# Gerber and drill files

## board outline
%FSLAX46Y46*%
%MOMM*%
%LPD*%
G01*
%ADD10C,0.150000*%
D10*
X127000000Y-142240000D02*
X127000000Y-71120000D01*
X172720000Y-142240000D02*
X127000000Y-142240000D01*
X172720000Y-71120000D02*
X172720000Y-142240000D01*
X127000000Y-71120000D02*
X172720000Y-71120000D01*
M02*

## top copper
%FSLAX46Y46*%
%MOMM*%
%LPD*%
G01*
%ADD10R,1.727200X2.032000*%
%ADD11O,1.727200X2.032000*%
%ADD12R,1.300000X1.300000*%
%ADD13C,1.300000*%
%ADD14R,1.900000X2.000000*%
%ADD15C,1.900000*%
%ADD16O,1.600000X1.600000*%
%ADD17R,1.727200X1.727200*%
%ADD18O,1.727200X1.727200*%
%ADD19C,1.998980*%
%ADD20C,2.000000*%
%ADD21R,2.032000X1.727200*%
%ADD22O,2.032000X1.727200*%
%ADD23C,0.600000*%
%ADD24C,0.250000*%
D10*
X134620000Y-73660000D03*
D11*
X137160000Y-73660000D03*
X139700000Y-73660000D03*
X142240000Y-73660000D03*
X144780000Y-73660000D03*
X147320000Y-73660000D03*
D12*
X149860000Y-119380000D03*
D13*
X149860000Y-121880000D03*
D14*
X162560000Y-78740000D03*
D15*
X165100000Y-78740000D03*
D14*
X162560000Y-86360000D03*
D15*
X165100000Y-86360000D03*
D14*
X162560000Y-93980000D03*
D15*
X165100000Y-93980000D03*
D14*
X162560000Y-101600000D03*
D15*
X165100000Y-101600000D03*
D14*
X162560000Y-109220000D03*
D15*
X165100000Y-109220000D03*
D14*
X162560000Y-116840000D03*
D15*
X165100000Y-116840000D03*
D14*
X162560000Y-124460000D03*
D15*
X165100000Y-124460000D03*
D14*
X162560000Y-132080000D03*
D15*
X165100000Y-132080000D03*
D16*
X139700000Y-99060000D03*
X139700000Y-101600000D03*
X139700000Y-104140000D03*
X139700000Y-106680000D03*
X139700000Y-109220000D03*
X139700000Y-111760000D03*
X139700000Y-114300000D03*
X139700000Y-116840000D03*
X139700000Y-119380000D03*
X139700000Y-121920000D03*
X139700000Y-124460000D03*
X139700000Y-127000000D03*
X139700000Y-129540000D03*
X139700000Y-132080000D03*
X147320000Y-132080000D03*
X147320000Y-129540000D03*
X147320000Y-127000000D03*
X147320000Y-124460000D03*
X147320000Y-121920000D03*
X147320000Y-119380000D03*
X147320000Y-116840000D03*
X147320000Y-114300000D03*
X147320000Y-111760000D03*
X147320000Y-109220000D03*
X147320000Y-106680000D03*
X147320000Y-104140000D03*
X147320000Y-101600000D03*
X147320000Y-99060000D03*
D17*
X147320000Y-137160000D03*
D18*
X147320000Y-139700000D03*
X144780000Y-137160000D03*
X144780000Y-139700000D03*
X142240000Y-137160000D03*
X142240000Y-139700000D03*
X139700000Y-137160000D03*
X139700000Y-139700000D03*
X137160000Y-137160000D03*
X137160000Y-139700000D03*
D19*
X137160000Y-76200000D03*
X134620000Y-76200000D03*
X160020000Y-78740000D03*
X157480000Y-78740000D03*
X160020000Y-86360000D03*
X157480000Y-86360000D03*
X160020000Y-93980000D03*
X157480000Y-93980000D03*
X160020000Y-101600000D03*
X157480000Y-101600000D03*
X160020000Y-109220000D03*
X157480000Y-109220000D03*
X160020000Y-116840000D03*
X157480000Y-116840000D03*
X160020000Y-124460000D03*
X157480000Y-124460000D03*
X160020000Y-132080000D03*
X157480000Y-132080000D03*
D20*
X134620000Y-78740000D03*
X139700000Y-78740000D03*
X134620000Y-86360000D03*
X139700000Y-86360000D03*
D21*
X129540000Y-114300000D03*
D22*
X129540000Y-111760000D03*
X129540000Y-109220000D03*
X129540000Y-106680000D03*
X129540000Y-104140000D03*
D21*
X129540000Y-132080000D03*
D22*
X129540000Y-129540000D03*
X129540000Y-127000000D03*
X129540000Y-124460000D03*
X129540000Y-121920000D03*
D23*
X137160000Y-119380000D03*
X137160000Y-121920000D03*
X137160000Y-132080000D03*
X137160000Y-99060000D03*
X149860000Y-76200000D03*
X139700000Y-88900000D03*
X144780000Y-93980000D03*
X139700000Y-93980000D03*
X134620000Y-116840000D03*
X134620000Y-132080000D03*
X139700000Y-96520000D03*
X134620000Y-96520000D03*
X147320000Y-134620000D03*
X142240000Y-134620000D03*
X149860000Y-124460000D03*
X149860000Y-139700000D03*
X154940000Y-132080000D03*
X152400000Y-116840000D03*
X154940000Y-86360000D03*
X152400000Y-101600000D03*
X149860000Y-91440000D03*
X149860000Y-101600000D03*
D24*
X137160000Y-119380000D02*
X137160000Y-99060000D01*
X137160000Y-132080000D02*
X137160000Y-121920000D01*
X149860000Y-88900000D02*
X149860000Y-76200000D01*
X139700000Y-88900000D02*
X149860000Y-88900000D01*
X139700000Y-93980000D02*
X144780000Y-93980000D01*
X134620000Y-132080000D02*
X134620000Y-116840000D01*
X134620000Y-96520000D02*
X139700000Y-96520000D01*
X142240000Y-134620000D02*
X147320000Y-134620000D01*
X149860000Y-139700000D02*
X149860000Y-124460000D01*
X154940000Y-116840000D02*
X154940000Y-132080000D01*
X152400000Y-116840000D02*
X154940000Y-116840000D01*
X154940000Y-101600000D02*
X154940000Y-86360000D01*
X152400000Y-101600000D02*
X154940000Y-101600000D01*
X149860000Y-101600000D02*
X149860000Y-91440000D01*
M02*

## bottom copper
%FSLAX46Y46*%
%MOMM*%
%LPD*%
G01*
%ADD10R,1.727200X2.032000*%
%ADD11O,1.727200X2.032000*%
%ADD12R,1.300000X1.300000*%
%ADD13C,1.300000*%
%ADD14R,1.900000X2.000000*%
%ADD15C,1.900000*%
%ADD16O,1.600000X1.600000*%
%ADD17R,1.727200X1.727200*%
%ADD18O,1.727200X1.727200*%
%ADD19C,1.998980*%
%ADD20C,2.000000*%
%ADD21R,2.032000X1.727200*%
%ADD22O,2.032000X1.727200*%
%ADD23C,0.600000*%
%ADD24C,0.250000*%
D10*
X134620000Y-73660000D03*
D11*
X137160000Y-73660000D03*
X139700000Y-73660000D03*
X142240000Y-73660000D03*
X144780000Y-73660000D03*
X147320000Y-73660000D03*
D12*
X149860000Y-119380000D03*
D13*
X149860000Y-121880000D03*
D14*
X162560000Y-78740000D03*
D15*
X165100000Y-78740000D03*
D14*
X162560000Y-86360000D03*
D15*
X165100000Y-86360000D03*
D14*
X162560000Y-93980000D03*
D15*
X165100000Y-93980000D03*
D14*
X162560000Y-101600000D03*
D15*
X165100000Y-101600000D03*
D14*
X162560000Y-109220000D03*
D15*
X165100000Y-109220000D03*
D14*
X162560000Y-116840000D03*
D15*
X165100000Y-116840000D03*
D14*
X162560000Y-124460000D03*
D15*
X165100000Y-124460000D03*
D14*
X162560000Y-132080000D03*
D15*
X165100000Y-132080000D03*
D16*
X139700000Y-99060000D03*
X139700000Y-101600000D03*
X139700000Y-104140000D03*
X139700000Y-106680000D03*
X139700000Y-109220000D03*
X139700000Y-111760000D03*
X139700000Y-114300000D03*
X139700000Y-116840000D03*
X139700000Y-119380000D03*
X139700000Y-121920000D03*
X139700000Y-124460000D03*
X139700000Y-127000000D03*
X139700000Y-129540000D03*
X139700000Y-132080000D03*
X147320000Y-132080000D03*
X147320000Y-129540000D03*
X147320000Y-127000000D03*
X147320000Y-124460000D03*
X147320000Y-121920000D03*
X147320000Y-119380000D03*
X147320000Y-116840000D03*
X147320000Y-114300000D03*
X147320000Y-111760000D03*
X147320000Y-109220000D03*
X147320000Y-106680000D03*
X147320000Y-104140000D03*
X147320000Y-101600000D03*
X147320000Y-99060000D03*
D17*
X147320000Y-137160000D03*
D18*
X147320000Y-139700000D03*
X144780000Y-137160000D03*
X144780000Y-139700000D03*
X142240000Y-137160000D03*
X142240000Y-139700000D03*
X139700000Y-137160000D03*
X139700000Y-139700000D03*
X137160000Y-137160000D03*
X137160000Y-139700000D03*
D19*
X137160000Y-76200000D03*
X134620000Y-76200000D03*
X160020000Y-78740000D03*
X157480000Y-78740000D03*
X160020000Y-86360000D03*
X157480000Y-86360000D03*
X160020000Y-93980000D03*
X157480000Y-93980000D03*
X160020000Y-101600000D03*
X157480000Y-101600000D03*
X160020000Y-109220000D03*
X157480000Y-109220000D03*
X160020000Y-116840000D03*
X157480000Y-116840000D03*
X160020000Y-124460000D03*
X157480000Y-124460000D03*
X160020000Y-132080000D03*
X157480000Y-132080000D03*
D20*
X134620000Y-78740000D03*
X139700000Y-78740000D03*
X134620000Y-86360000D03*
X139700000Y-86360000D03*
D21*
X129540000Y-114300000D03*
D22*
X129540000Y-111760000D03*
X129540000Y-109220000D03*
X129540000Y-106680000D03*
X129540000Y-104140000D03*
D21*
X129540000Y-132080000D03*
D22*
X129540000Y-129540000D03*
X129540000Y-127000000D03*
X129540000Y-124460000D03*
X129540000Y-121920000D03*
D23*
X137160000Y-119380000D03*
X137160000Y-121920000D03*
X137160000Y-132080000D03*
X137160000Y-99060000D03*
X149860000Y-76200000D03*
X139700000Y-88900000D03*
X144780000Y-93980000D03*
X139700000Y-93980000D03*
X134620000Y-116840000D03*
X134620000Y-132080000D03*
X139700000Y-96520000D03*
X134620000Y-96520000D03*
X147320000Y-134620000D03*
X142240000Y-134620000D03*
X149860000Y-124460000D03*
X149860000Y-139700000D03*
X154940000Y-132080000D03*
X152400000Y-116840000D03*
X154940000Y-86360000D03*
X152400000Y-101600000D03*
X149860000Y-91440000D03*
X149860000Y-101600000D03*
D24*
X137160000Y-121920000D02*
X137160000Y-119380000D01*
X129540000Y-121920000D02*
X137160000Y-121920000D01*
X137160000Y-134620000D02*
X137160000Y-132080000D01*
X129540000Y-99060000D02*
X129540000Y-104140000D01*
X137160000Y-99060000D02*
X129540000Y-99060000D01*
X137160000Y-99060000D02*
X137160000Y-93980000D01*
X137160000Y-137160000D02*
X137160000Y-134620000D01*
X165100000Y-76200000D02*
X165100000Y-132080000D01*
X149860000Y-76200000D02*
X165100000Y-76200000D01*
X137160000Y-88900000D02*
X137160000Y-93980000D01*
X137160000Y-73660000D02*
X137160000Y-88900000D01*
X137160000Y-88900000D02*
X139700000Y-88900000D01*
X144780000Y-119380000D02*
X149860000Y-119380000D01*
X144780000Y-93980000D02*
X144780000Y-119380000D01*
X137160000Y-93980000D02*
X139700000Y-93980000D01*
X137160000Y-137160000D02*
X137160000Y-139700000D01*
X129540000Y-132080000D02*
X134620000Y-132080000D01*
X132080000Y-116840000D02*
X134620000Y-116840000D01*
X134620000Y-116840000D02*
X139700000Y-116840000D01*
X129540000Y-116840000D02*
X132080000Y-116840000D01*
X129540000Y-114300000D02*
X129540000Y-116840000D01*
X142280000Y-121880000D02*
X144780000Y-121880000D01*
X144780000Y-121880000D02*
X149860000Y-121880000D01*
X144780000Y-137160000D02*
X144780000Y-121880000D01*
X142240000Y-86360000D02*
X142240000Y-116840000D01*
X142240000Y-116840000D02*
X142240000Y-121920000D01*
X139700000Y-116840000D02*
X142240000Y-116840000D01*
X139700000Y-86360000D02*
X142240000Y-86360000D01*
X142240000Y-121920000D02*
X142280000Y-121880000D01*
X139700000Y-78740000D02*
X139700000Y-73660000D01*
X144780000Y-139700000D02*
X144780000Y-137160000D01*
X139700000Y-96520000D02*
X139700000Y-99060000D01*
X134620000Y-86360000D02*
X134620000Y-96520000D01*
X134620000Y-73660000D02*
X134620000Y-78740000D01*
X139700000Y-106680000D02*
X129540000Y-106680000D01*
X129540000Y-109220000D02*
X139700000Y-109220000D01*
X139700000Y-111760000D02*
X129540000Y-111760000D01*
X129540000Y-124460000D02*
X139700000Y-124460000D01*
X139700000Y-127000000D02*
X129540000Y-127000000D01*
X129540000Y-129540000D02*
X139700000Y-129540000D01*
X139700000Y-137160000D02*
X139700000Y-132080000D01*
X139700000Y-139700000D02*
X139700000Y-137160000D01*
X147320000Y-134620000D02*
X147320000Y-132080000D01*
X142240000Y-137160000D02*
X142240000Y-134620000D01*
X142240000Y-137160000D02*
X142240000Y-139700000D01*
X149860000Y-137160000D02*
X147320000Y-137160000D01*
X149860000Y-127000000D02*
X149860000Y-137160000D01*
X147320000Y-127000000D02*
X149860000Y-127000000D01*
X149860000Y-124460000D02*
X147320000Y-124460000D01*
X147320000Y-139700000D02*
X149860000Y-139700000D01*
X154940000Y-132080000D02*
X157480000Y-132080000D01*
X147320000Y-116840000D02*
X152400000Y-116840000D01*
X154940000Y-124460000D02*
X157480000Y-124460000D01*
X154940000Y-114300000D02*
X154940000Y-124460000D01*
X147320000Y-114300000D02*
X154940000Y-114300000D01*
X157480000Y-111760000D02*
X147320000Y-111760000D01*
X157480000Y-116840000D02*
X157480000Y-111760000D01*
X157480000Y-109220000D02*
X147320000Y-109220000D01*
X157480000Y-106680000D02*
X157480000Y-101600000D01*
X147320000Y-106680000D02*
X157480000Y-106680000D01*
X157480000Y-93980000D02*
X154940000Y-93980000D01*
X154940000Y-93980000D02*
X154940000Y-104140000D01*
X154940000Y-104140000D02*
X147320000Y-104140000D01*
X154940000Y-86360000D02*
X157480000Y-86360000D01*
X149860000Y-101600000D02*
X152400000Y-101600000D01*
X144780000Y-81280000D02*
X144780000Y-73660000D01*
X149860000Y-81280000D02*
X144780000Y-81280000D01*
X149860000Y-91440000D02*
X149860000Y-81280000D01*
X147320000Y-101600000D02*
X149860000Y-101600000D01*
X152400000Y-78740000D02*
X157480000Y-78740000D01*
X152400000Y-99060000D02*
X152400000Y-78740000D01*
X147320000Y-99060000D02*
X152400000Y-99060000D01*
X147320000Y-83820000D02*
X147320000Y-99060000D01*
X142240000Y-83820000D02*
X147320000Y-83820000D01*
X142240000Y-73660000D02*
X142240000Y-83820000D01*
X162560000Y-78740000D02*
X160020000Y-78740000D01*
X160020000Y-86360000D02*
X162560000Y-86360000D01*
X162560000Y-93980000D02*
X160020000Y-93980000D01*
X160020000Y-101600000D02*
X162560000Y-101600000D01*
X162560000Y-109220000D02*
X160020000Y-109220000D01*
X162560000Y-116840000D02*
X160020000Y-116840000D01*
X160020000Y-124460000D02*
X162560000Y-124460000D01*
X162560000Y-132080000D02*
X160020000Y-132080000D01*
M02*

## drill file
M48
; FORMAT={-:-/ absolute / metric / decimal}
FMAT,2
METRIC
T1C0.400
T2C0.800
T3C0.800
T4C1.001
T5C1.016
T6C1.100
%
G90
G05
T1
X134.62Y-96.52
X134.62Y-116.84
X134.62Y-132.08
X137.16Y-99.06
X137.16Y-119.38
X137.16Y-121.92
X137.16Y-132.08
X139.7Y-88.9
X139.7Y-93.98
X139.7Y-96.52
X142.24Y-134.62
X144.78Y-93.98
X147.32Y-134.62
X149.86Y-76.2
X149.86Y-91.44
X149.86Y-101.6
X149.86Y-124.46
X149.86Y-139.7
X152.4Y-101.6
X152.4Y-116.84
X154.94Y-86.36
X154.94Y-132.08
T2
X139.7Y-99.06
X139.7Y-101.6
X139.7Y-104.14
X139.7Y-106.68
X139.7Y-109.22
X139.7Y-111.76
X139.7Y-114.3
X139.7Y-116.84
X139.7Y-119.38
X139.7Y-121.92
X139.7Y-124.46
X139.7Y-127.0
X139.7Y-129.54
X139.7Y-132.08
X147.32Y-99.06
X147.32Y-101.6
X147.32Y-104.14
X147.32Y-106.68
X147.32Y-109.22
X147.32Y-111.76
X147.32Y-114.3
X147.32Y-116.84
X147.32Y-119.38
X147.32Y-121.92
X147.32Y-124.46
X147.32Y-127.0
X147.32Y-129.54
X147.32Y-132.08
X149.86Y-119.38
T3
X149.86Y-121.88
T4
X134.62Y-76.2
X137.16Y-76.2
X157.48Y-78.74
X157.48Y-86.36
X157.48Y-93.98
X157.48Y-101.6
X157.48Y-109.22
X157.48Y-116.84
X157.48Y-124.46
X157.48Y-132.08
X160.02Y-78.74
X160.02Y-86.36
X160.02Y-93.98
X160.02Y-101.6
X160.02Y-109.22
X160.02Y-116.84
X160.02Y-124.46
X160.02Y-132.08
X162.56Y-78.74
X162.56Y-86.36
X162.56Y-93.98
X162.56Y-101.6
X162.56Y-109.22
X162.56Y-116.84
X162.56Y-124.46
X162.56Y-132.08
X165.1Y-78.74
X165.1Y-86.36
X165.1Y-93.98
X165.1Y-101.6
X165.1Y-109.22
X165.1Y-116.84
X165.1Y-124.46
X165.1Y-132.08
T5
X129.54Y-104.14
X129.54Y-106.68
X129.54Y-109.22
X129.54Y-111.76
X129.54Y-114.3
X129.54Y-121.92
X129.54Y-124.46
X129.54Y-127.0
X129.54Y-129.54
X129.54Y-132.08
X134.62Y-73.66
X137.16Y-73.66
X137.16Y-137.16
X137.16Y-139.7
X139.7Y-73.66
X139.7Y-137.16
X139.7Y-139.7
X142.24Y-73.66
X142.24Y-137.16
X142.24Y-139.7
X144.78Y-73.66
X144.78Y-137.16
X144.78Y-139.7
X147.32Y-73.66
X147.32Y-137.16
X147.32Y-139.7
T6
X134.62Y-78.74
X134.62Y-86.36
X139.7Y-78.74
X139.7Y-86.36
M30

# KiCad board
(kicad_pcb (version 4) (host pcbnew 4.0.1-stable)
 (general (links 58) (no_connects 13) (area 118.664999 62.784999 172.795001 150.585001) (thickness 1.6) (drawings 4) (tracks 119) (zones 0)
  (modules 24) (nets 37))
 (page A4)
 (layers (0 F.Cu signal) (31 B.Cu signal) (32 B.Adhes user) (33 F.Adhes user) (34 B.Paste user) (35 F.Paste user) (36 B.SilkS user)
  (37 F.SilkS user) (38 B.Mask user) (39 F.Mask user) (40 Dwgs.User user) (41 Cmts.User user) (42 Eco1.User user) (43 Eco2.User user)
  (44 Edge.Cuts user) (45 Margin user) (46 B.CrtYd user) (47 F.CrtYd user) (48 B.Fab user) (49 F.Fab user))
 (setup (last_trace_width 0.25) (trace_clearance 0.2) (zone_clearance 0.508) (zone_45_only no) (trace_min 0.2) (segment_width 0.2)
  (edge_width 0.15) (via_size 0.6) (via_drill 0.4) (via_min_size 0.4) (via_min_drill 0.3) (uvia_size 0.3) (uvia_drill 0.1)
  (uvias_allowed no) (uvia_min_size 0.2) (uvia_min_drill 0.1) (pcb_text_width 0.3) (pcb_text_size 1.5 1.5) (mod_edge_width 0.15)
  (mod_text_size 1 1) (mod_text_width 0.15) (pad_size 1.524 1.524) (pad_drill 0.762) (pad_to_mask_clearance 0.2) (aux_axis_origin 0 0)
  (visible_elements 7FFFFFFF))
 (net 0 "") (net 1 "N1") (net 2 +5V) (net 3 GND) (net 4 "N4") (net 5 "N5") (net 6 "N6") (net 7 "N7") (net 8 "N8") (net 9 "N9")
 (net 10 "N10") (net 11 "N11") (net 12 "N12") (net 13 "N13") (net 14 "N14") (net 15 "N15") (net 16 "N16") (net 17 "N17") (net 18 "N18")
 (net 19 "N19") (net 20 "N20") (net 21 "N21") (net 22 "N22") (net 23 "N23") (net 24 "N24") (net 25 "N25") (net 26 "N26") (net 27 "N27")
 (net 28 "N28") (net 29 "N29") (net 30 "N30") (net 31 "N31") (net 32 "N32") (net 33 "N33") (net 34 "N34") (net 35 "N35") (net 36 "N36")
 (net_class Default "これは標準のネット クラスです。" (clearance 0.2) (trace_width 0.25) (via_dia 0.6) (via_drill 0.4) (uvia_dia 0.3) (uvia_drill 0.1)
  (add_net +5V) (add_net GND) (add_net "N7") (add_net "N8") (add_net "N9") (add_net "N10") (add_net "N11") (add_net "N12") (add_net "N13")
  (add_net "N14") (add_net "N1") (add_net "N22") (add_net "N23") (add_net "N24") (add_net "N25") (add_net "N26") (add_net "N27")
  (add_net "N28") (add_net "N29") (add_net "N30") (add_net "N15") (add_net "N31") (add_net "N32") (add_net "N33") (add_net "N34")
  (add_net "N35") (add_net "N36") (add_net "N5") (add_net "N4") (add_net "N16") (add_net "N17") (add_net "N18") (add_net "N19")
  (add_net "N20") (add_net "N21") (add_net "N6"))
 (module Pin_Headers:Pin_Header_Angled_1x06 (layer F.Cu) (at 134.62 73.66 90)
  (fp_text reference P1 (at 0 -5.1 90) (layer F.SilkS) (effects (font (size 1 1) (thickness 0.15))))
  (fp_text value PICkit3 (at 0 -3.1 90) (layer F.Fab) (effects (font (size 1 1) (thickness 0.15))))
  (pad 1 thru_hole rect (at 0 0 90) (size 2.032 1.7272) (drill 1.016) (layers *.Cu *.Mask) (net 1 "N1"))
  (pad 2 thru_hole oval (at 0 2.54 90) (size 2.032 1.7272) (drill 1.016) (layers *.Cu *.Mask) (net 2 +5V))
  (pad 3 thru_hole oval (at 0 5.08 90) (size 2.032 1.7272) (drill 1.016) (layers *.Cu *.Mask) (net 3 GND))
  (pad 4 thru_hole oval (at 0 7.62 90) (size 2.032 1.7272) (drill 1.016) (layers *.Cu *.Mask) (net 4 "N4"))
  (pad 5 thru_hole oval (at 0 10.16 90) (size 2.032 1.7272) (drill 1.016) (layers *.Cu *.Mask) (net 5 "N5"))
  (pad 6 thru_hole oval (at 0 12.7 90) (size 2.032 1.7272) (drill 1.016) (layers *.Cu *.Mask) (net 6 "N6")))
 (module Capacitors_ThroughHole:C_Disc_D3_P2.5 (layer F.Cu) (at 149.86 119.38 270)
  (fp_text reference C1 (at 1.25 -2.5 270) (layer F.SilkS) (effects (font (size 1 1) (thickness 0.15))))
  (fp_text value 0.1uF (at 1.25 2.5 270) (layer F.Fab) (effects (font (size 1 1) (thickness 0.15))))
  (pad 1 thru_hole rect (at 0 0 270) (size 1.3 1.3) (drill 0.8) (layers *.Cu *.Mask) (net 2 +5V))
  (pad 2 thru_hole circle (at 2.5 0 270) (size 1.3 1.3) (drill 0.8001) (layers *.Cu *.Mask) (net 3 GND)))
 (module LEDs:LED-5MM (layer F.Cu) (at 162.56 78.74)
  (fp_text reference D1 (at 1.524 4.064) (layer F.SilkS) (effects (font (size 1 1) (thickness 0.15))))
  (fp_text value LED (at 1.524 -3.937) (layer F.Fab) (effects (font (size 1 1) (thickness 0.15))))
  (pad 1 thru_hole rect (at 0 0 90) (size 2 1.9) (drill 1.00076) (layers *.Cu *.Mask) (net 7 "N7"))
  (pad 2 thru_hole circle (at 2.54 0) (size 1.9 1.9) (drill 1.00076) (layers *.Cu *.Mask) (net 2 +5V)))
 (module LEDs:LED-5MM (layer F.Cu) (at 162.56 86.36)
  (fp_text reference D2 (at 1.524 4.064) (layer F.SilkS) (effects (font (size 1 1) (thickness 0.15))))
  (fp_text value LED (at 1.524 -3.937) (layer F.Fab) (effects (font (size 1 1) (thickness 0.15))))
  (pad 1 thru_hole rect (at 0 0 90) (size 2 1.9) (drill 1.00076) (layers *.Cu *.Mask) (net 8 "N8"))
  (pad 2 thru_hole circle (at 2.54 0) (size 1.9 1.9) (drill 1.00076) (layers *.Cu *.Mask) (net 2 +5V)))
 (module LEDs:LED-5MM (layer F.Cu) (at 162.56 93.98)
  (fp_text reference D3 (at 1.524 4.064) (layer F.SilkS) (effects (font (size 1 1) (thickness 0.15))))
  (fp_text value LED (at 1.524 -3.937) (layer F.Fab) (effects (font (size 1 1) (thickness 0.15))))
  (pad 1 thru_hole rect (at 0 0 90) (size 2 1.9) (drill 1.00076) (layers *.Cu *.Mask) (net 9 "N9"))
  (pad 2 thru_hole circle (at 2.54 0) (size 1.9 1.9) (drill 1.00076) (layers *.Cu *.Mask) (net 2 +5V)))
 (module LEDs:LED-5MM (layer F.Cu) (at 162.56 101.6)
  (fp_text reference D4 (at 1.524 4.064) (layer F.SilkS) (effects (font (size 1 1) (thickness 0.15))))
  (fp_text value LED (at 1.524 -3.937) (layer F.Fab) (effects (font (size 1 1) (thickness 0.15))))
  (pad 1 thru_hole rect (at 0 0 90) (size 2 1.9) (drill 1.00076) (layers *.Cu *.Mask) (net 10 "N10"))
  (pad 2 thru_hole circle (at 2.54 0) (size 1.9 1.9) (drill 1.00076) (layers *.Cu *.Mask) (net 2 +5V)))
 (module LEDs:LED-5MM (layer F.Cu) (at 162.56 109.22)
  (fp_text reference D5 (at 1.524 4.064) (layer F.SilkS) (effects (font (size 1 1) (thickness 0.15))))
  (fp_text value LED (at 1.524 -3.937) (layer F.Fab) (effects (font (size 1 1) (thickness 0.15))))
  (pad 1 thru_hole rect (at 0 0 90) (size 2 1.9) (drill 1.00076) (layers *.Cu *.Mask) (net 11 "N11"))
  (pad 2 thru_hole circle (at 2.54 0) (size 1.9 1.9) (drill 1.00076) (layers *.Cu *.Mask) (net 2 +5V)))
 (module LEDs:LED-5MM (layer F.Cu) (at 162.56 116.84)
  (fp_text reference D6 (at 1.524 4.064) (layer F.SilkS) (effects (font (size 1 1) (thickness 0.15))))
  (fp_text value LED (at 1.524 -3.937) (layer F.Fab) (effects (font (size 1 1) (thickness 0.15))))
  (pad 1 thru_hole rect (at 0 0 90) (size 2 1.9) (drill 1.00076) (layers *.Cu *.Mask) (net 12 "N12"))
  (pad 2 thru_hole circle (at 2.54 0) (size 1.9 1.9) (drill 1.00076) (layers *.Cu *.Mask) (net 2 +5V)))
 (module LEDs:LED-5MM (layer F.Cu) (at 162.56 124.46)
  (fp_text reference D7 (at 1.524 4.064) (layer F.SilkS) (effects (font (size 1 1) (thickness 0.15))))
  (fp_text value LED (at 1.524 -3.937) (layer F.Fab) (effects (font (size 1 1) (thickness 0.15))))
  (pad 1 thru_hole rect (at 0 0 90) (size 2 1.9) (drill 1.00076) (layers *.Cu *.Mask) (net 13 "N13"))
  (pad 2 thru_hole circle (at 2.54 0) (size 1.9 1.9) (drill 1.00076) (layers *.Cu *.Mask) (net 2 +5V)))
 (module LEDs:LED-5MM (layer F.Cu) (at 162.56 132.08)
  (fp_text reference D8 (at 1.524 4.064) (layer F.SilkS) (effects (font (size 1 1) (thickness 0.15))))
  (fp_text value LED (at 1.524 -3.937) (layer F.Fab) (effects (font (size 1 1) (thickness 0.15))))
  (pad 1 thru_hole rect (at 0 0 90) (size 2 1.9) (drill 1.00076) (layers *.Cu *.Mask) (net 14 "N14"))
  (pad 2 thru_hole circle (at 2.54 0) (size 1.9 1.9) (drill 1.00076) (layers *.Cu *.Mask) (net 2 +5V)))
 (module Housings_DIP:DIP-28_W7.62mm (layer F.Cu) (at 139.7 99.06)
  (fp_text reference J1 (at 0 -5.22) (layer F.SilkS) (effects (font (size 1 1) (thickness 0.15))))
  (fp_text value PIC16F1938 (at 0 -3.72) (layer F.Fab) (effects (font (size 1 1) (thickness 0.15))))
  (pad 1 thru_hole oval (at 0 0) (size 1.6 1.6) (drill 0.8) (layers *.Cu *.Mask) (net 1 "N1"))
  (pad 2 thru_hole oval (at 0 2.54) (size 1.6 1.6) (drill 0.8) (layers *.Cu *.Mask) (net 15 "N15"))
  (pad 3 thru_hole oval (at 0 5.08) (size 1.6 1.6) (drill 0.8) (layers *.Cu *.Mask) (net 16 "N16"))
  (pad 4 thru_hole oval (at 0 7.62) (size 1.6 1.6) (drill 0.8) (layers *.Cu *.Mask) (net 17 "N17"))
  (pad 5 thru_hole oval (at 0 10.16) (size 1.6 1.6) (drill 0.8) (layers *.Cu *.Mask) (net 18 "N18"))
  (pad 6 thru_hole oval (at 0 12.7) (size 1.6 1.6) (drill 0.8) (layers *.Cu *.Mask) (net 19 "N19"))
  (pad 7 thru_hole oval (at 0 15.24) (size 1.6 1.6) (drill 0.8) (layers *.Cu *.Mask) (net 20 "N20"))
  (pad 8 thru_hole oval (at 0 17.78) (size 1.6 1.6) (drill 0.8) (layers *.Cu *.Mask) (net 3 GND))
  (pad 9 thru_hole oval (at 0 20.32) (size 1.6 1.6) (drill 0.8) (layers *.Cu *.Mask) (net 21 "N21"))
  (pad 10 thru_hole oval (at 0 22.86) (size 1.6 1.6) (drill 0.8) (layers *.Cu *.Mask) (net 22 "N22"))
  (pad 11 thru_hole oval (at 0 25.4) (size 1.6 1.6) (drill 0.8) (layers *.Cu *.Mask) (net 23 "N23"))
  (pad 12 thru_hole oval (at 0 27.94) (size 1.6 1.6) (drill 0.8) (layers *.Cu *.Mask) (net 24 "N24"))
  (pad 13 thru_hole oval (at 0 30.48) (size 1.6 1.6) (drill 0.8) (layers *.Cu *.Mask) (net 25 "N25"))
  (pad 14 thru_hole oval (at 0 33.02) (size 1.6 1.6) (drill 0.8) (layers *.Cu *.Mask) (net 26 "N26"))
  (pad 15 thru_hole oval (at 7.62 33.02) (size 1.6 1.6) (drill 0.8) (layers *.Cu *.Mask) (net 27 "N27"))
  (pad 16 thru_hole oval (at 7.62 30.48) (size 1.6 1.6) (drill 0.8) (layers *.Cu *.Mask) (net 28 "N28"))
  (pad 17 thru_hole oval (at 7.62 27.94) (size 1.6 1.6) (drill 0.8) (layers *.Cu *.Mask) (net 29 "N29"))
  (pad 18 thru_hole oval (at 7.62 25.4) (size 1.6 1.6) (drill 0.8) (layers *.Cu *.Mask) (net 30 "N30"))
  (pad 19 thru_hole oval (at 7.62 22.86) (size 1.6 1.6) (drill 0.8) (layers *.Cu *.Mask) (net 3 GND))
  (pad 20 thru_hole oval (at 7.62 20.32) (size 1.6 1.6) (drill 0.8) (layers *.Cu *.Mask) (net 2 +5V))
  (pad 21 thru_hole oval (at 7.62 17.78) (size 1.6 1.6) (drill 0.8) (layers *.Cu *.Mask) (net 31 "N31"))
  (pad 22 thru_hole oval (at 7.62 15.24) (size 1.6 1.6) (drill 0.8) (layers *.Cu *.Mask) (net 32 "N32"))
  (pad 23 thru_hole oval (at 7.62 12.7) (size 1.6 1.6) (drill 0.8) (layers *.Cu *.Mask) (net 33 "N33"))
  (pad 24 thru_hole oval (at 7.62 10.16) (size 1.6 1.6) (drill 0.8) (layers *.Cu *.Mask) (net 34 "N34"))
  (pad 25 thru_hole oval (at 7.62 7.62) (size 1.6 1.6) (drill 0.8) (layers *.Cu *.Mask) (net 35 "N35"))
  (pad 26 thru_hole oval (at 7.62 5.08) (size 1.6 1.6) (drill 0.8) (layers *.Cu *.Mask) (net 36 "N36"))
  (pad 27 thru_hole oval (at 7.62 2.54) (size 1.6 1.6) (drill 0.8) (layers *.Cu *.Mask) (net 5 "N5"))
  (pad 28 thru_hole oval (at 7.62 0) (size 1.6 1.6) (drill 0.8) (layers *.Cu *.Mask) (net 4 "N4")))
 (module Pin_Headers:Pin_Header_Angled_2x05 (layer F.Cu) (at 147.32 137.16 270)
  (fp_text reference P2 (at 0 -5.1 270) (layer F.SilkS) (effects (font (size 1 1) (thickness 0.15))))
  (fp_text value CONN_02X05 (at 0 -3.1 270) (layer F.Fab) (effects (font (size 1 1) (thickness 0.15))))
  (pad 1 thru_hole rect (at 0 0 270) (size 1.7272 1.7272) (drill 1.016) (layers *.Cu *.Mask) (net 29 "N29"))
  (pad 2 thru_hole oval (at 2.54 0 270) (size 1.7272 1.7272) (drill 1.016) (layers *.Cu *.Mask) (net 30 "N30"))
  (pad 3 thru_hole oval (at 0 2.54 270) (size 1.7272 1.7272) (drill 1.016) (layers *.Cu *.Mask) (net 3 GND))
  (pad 4 thru_hole oval (at 2.54 2.54 270) (size 1.7272 1.7272) (drill 1.016) (layers *.Cu *.Mask) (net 3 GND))
  (pad 5 thru_hole oval (at 0 5.08 270) (size 1.7272 1.7272) (drill 1.016) (layers *.Cu *.Mask) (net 27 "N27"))
  (pad 6 thru_hole oval (at 2.54 5.08 270) (size 1.7272 1.7272) (drill 1.016) (layers *.Cu *.Mask) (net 27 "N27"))
  (pad 7 thru_hole oval (at 0 7.62 270) (size 1.7272 1.7272) (drill 1.016) (layers *.Cu *.Mask) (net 26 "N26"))
  (pad 8 thru_hole oval (at 2.54 7.62 270) (size 1.7272 1.7272) (drill 1.016) (layers *.Cu *.Mask) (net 26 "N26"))
  (pad 9 thru_hole oval (at 0 10.16 270) (size 1.7272 1.7272) (drill 1.016) (layers *.Cu *.Mask) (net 2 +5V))
  (pad 10 thru_hole oval (at 2.54 10.16 270) (size 1.7272 1.7272) (drill 1.016) (layers *.Cu *.Mask) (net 2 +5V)))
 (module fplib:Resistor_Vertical (layer F.Cu) (at 135.89 76.2 180)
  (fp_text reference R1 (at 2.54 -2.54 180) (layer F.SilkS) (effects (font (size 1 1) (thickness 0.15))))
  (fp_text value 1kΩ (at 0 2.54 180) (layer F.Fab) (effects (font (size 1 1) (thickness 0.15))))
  (pad 1 thru_hole circle (at -1.27 0 180) (size 1.99898 1.99898) (drill 1.00076) (layers *.Cu *.SilkS *.Mask) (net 2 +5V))
  (pad 2 thru_hole circle (at 1.27 0 180) (size 1.99898 1.99898) (drill 1.00076) (layers *.Cu *.SilkS *.Mask) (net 1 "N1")))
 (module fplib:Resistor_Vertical (layer F.Cu) (at 158.75 78.74 180)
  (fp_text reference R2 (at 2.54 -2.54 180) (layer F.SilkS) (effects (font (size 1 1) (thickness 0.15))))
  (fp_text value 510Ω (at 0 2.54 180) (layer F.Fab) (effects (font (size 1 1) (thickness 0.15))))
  (pad 1 thru_hole circle (at -1.27 0 180) (size 1.99898 1.99898) (drill 1.00076) (layers *.Cu *.SilkS *.Mask) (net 7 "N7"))
  (pad 2 thru_hole circle (at 1.27 0 180) (size 1.99898 1.99898) (drill 1.00076) (layers *.Cu *.SilkS *.Mask) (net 4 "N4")))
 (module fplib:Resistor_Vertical (layer F.Cu) (at 158.75 86.36 180)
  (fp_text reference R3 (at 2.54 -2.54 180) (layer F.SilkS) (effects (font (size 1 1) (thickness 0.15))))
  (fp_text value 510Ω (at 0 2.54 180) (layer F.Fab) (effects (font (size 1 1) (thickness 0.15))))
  (pad 1 thru_hole circle (at -1.27 0 180) (size 1.99898 1.99898) (drill 1.00076) (layers *.Cu *.SilkS *.Mask) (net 8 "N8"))
  (pad 2 thru_hole circle (at 1.27 0 180) (size 1.99898 1.99898) (drill 1.00076) (layers *.Cu *.SilkS *.Mask) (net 5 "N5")))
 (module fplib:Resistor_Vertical (layer F.Cu) (at 158.75 93.98 180)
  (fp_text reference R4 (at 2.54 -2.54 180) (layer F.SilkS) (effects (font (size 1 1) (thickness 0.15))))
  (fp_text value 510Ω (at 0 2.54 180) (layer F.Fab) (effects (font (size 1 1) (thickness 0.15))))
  (pad 1 thru_hole circle (at -1.27 0 180) (size 1.99898 1.99898) (drill 1.00076) (layers *.Cu *.SilkS *.Mask) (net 9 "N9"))
  (pad 2 thru_hole circle (at 1.27 0 180) (size 1.99898 1.99898) (drill 1.00076) (layers *.Cu *.SilkS *.Mask) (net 36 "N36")))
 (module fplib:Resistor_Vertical (layer F.Cu) (at 158.75 101.6 180)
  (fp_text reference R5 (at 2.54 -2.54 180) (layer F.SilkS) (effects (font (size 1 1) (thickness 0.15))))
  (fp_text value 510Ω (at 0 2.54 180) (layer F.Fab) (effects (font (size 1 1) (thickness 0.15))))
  (pad 1 thru_hole circle (at -1.27 0 180) (size 1.99898 1.99898) (drill 1.00076) (layers *.Cu *.SilkS *.Mask) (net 10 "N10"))
  (pad 2 thru_hole circle (at 1.27 0 180) (size 1.99898 1.99898) (drill 1.00076) (layers *.Cu *.SilkS *.Mask) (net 35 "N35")))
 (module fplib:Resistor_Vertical (layer F.Cu) (at 158.75 109.22 180)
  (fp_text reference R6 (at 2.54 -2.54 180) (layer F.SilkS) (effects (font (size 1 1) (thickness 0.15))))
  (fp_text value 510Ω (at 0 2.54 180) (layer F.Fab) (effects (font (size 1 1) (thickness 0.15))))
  (pad 1 thru_hole circle (at -1.27 0 180) (size 1.99898 1.99898) (drill 1.00076) (layers *.Cu *.SilkS *.Mask) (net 11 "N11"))
  (pad 2 thru_hole circle (at 1.27 0 180) (size 1.99898 1.99898) (drill 1.00076) (layers *.Cu *.SilkS *.Mask) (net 34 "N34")))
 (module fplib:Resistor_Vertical (layer F.Cu) (at 158.75 116.84 180)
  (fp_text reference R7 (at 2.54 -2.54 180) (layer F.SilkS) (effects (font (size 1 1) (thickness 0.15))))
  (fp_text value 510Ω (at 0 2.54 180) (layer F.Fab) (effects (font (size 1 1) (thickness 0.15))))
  (pad 1 thru_hole circle (at -1.27 0 180) (size 1.99898 1.99898) (drill 1.00076) (layers *.Cu *.SilkS *.Mask) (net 12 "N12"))
  (pad 2 thru_hole circle (at 1.27 0 180) (size 1.99898 1.99898) (drill 1.00076) (layers *.Cu *.SilkS *.Mask) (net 33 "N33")))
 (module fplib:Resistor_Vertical (layer F.Cu) (at 158.75 124.46 180)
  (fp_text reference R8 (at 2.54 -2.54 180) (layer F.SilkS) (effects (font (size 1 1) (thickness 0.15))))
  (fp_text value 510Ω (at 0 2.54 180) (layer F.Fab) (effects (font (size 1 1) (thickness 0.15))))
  (pad 1 thru_hole circle (at -1.27 0 180) (size 1.99898 1.99898) (drill 1.00076) (layers *.Cu *.SilkS *.Mask) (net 13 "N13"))
  (pad 2 thru_hole circle (at 1.27 0 180) (size 1.99898 1.99898) (drill 1.00076) (layers *.Cu *.SilkS *.Mask) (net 32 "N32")))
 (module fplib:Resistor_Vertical (layer F.Cu) (at 158.75 132.08 180)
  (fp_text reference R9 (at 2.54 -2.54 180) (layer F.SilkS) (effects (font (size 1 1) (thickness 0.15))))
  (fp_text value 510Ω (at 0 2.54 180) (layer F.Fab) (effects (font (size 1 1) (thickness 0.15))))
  (pad 1 thru_hole circle (at -1.27 0 180) (size 1.99898 1.99898) (drill 1.00076) (layers *.Cu *.SilkS *.Mask) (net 14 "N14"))
  (pad 2 thru_hole circle (at 1.27 0 180) (size 1.99898 1.99898) (drill 1.00076) (layers *.Cu *.SilkS *.Mask) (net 31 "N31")))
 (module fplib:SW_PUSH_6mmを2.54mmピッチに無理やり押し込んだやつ (layer F.Cu) (at 137.16 82.55 270)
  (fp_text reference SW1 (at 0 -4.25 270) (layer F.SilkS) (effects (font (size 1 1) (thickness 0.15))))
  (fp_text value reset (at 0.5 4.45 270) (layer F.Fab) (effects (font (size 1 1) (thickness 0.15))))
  (pad 2 thru_hole circle (at -3.81 2.54) (size 2 2) (drill 1.1) (layers *.Cu *.Mask) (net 1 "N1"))
  (pad 1 thru_hole circle (at -3.81 -2.54) (size 2 2) (drill 1.1) (layers *.Cu *.Mask) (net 3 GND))
  (pad 2 thru_hole circle (at 3.81 2.54) (size 2 2) (drill 1.1) (layers *.Cu *.Mask) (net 1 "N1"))
  (pad 1 thru_hole circle (at 3.81 -2.54) (size 2 2) (drill 1.1) (layers *.Cu *.Mask) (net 3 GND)))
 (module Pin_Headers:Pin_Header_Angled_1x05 (layer F.Cu) (at 129.54 114.3 180)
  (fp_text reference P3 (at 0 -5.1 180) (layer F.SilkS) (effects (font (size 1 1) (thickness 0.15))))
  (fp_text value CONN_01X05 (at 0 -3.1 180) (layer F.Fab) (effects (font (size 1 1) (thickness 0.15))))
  (pad 1 thru_hole rect (at 0 0 180) (size 2.032 1.7272) (drill 1.016) (layers *.Cu *.Mask F.SilkS) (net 3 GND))
  (pad 2 thru_hole oval (at 0 2.54 180) (size 2.032 1.7272) (drill 1.016) (layers *.Cu *.Mask F.SilkS) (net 19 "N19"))
  (pad 3 thru_hole oval (at 0 5.08 180) (size 2.032 1.7272) (drill 1.016) (layers *.Cu *.Mask F.SilkS) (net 18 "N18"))
  (pad 4 thru_hole oval (at 0 7.62 180) (size 2.032 1.7272) (drill 1.016) (layers *.Cu *.Mask F.SilkS) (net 17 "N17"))
  (pad 5 thru_hole oval (at 0 10.16 180) (size 2.032 1.7272) (drill 1.016) (layers *.Cu *.Mask F.SilkS) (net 2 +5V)))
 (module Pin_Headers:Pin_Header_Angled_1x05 (layer F.Cu) (at 129.54 132.08 180)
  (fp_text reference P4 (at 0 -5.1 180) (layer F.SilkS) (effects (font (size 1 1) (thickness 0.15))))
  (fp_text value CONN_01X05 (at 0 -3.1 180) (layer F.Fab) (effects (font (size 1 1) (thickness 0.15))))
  (pad 1 thru_hole rect (at 0 0 180) (size 2.032 1.7272) (drill 1.016) (layers *.Cu *.Mask F.SilkS) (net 3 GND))
  (pad 2 thru_hole oval (at 0 2.54 180) (size 2.032 1.7272) (drill 1.016) (layers *.Cu *.Mask F.SilkS) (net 25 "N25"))
  (pad 3 thru_hole oval (at 0 5.08 180) (size 2.032 1.7272) (drill 1.016) (layers *.Cu *.Mask F.SilkS) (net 24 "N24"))
  (pad 4 thru_hole oval (at 0 7.62 180) (size 2.032 1.7272) (drill 1.016) (layers *.Cu *.Mask F.SilkS) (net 23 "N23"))
  (pad 5 thru_hole oval (at 0 10.16 180) (size 2.032 1.7272) (drill 1.016) (layers *.Cu *.Mask F.SilkS) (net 2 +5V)))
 (gr_line (start 127 142.24) (end 127 71.12) (layer Edge.Cuts) (width 0.15))
 (gr_line (start 172.72 142.24) (end 127 142.24) (layer Edge.Cuts) (width 0.15))
 (gr_line (start 172.72 71.12) (end 172.72 142.24) (layer Edge.Cuts) (width 0.15))
 (gr_line (start 127 71.12) (end 172.72 71.12) (layer Edge.Cuts) (width 0.15))
 (segment (start 137.16 121.92) (end 137.16 119.38) (width 0.25) (layer B.Cu) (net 2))
 (via (at 137.16 119.38) (size 0.6) (drill 0.4) (layers F.Cu B.Cu) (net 2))
 (segment (start 129.54 121.92) (end 137.16 121.92) (width 0.25) (layer B.Cu) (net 2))
 (segment (start 137.16 119.38) (end 137.16 99.06) (width 0.25) (layer F.Cu) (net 2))
 (segment (start 137.16 132.08) (end 137.16 121.92) (width 0.25) (layer F.Cu) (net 2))
 (via (at 137.16 121.92) (size 0.6) (drill 0.4) (layers F.Cu B.Cu) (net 2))
 (segment (start 137.16 134.62) (end 137.16 132.08) (width 0.25) (layer B.Cu) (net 2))
 (via (at 137.16 132.08) (size 0.6) (drill 0.4) (layers F.Cu B.Cu) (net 2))
 (segment (start 129.54 99.06) (end 129.54 104.14) (width 0.25) (layer B.Cu) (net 2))
 (segment (start 137.16 99.06) (end 129.54 99.06) (width 0.25) (layer B.Cu) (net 2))
 (segment (start 137.16 99.06) (end 137.16 93.98) (width 0.25) (layer B.Cu) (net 2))
 (via (at 137.16 99.06) (size 0.6) (drill 0.4) (layers F.Cu B.Cu) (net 2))
 (segment (start 137.16 137.16) (end 137.16 134.62) (width 0.25) (layer B.Cu) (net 2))
 (segment (start 165.1 76.2) (end 165.1 132.08) (width 0.25) (layer B.Cu) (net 2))
 (segment (start 149.86 76.2) (end 165.1 76.2) (width 0.25) (layer B.Cu) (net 2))
 (segment (start 149.86 88.9) (end 149.86 76.2) (width 0.25) (layer F.Cu) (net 2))
 (via (at 149.86 76.2) (size 0.6) (drill 0.4) (layers F.Cu B.Cu) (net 2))
 (segment (start 139.7 88.9) (end 149.86 88.9) (width 0.25) (layer F.Cu) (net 2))
 (segment (start 137.16 88.9) (end 137.16 93.98) (width 0.25) (layer B.Cu) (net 2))
 (segment (start 137.16 73.66) (end 137.16 88.9) (width 0.25) (layer B.Cu) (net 2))
 (segment (start 137.16 88.9) (end 139.7 88.9) (width 0.25) (layer B.Cu) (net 2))
 (via (at 139.7 88.9) (size 0.6) (drill 0.4) (layers F.Cu B.Cu) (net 2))
 (segment (start 144.78 119.38) (end 149.86 119.38) (width 0.25) (layer B.Cu) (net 2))
 (segment (start 144.78 93.98) (end 144.78 119.38) (width 0.25) (layer B.Cu) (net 2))
 (segment (start 139.7 93.98) (end 144.78 93.98) (width 0.25) (layer F.Cu) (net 2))
 (via (at 144.78 93.98) (size 0.6) (drill 0.4) (layers F.Cu B.Cu) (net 2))
 (segment (start 137.16 93.98) (end 139.7 93.98) (width 0.25) (layer B.Cu) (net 2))
 (via (at 139.7 93.98) (size 0.6) (drill 0.4) (layers F.Cu B.Cu) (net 2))
 (segment (start 137.16 137.16) (end 137.16 139.7) (width 0.25) (layer B.Cu) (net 2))
 (segment (start 134.62 132.08) (end 134.62 116.84) (width 0.25) (layer F.Cu) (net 3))
 (via (at 134.62 116.84) (size 0.6) (drill 0.4) (layers F.Cu B.Cu) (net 3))
 (segment (start 129.54 132.08) (end 134.62 132.08) (width 0.25) (layer B.Cu) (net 3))
 (via (at 134.62 132.08) (size 0.6) (drill 0.4) (layers F.Cu B.Cu) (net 3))
 (segment (start 132.08 116.84) (end 134.62 116.84) (width 0.25) (layer B.Cu) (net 3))
 (segment (start 134.62 116.84) (end 139.7 116.84) (width 0.25) (layer B.Cu) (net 3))
 (segment (start 129.54 116.84) (end 132.08 116.84) (width 0.25) (layer B.Cu) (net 3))
 (segment (start 129.54 114.3) (end 129.54 116.84) (width 0.25) (layer B.Cu) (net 3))
 (segment (start 142.28 121.88) (end 144.78 121.88) (width 0.25) (layer B.Cu) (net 3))
 (segment (start 144.78 121.88) (end 149.86 121.88) (width 0.25) (layer B.Cu) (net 3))
 (segment (start 144.78 137.16) (end 144.78 121.88) (width 0.25) (layer B.Cu) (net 3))
 (segment (start 142.24 86.36) (end 142.24 116.84) (width 0.25) (layer B.Cu) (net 3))
 (segment (start 142.24 116.84) (end 142.24 121.92) (width 0.25) (layer B.Cu) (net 3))
 (segment (start 139.7 116.84) (end 142.24 116.84) (width 0.25) (layer B.Cu) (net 3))
 (segment (start 139.7 86.36) (end 142.24 86.36) (width 0.25) (layer B.Cu) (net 3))
 (segment (start 142.24 121.92) (end 142.28 121.88) (width 0.25) (layer B.Cu) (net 3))
 (segment (start 139.7 78.74) (end 139.7 73.66) (width 0.25) (layer B.Cu) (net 3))
 (segment (start 144.78 139.7) (end 144.78 137.16) (width 0.25) (layer B.Cu) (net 3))
 (segment (start 139.7 96.52) (end 139.7 99.06) (width 0.25) (layer B.Cu) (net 1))
 (segment (start 134.62 96.52) (end 139.7 96.52) (width 0.25) (layer F.Cu) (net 1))
 (via (at 139.7 96.52) (size 0.6) (drill 0.4) (layers F.Cu B.Cu) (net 1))
 (segment (start 134.62 86.36) (end 134.62 96.52) (width 0.25) (layer B.Cu) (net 1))
 (via (at 134.62 96.52) (size 0.6) (drill 0.4) (layers F.Cu B.Cu) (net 1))
 (segment (start 134.62 73.66) (end 134.62 78.74) (width 0.25) (layer B.Cu) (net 1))
 (segment (start 139.7 106.68) (end 129.54 106.68) (width 0.25) (layer B.Cu) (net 17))
 (segment (start 129.54 109.22) (end 139.7 109.22) (width 0.25) (layer B.Cu) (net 18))
 (segment (start 139.7 111.76) (end 129.54 111.76) (width 0.25) (layer B.Cu) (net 19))
 (segment (start 129.54 124.46) (end 139.7 124.46) (width 0.25) (layer B.Cu) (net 23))
 (segment (start 139.7 127) (end 129.54 127) (width 0.25) (layer B.Cu) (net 24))
 (segment (start 129.54 129.54) (end 139.7 129.54) (width 0.25) (layer B.Cu) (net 25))
 (segment (start 139.7 137.16) (end 139.7 132.08) (width 0.25) (layer B.Cu) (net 26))
 (segment (start 139.7 139.7) (end 139.7 137.16) (width 0.25) (layer B.Cu) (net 26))
 (segment (start 147.32 134.62) (end 147.32 132.08) (width 0.25) (layer B.Cu) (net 27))
 (segment (start 142.24 134.62) (end 147.32 134.62) (width 0.25) (layer F.Cu) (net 27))
 (via (at 147.32 134.62) (size 0.6) (drill 0.4) (layers F.Cu B.Cu) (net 27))
 (segment (start 142.24 137.16) (end 142.24 134.62) (width 0.25) (layer B.Cu) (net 27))
 (via (at 142.24 134.62) (size 0.6) (drill 0.4) (layers F.Cu B.Cu) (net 27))
 (segment (start 142.24 137.16) (end 142.24 139.7) (width 0.25) (layer B.Cu) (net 27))
 (segment (start 149.86 137.16) (end 147.32 137.16) (width 0.25) (layer B.Cu) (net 29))
 (segment (start 149.86 127) (end 149.86 137.16) (width 0.25) (layer B.Cu) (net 29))
 (segment (start 147.32 127) (end 149.86 127) (width 0.25) (layer B.Cu) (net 29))
 (segment (start 149.86 124.46) (end 147.32 124.46) (width 0.25) (layer B.Cu) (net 30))
 (segment (start 149.86 139.7) (end 149.86 124.46) (width 0.25) (layer F.Cu) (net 30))
 (via (at 149.86 124.46) (size 0.6) (drill 0.4) (layers F.Cu B.Cu) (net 30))
 (segment (start 147.32 139.7) (end 149.86 139.7) (width 0.25) (layer B.Cu) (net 30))
 (via (at 149.86 139.7) (size 0.6) (drill 0.4) (layers F.Cu B.Cu) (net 30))
 (segment (start 154.94 132.08) (end 157.48 132.08) (width 0.25) (layer B.Cu) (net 31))
 (segment (start 154.94 116.84) (end 154.94 132.08) (width 0.25) (layer F.Cu) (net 31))
 (via (at 154.94 132.08) (size 0.6) (drill 0.4) (layers F.Cu B.Cu) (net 31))
 (segment (start 152.4 116.84) (end 154.94 116.84) (width 0.25) (layer F.Cu) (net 31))
 (segment (start 147.32 116.84) (end 152.4 116.84) (width 0.25) (layer B.Cu) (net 31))
 (via (at 152.4 116.84) (size 0.6) (drill 0.4) (layers F.Cu B.Cu) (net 31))
 (segment (start 154.94 124.46) (end 157.48 124.46) (width 0.25) (layer B.Cu) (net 32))
 (segment (start 154.94 114.3) (end 154.94 124.46) (width 0.25) (layer B.Cu) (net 32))
 (segment (start 147.32 114.3) (end 154.94 114.3) (width 0.25) (layer B.Cu) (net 32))
 (segment (start 157.48 111.76) (end 147.32 111.76) (width 0.25) (layer B.Cu) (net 33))
 (segment (start 157.48 116.84) (end 157.48 111.76) (width 0.25) (layer B.Cu) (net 33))
 (segment (start 157.48 109.22) (end 147.32 109.22) (width 0.25) (layer B.Cu) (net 34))
 (segment (start 157.48 106.68) (end 157.48 101.6) (width 0.25) (layer B.Cu) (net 35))
 (segment (start 147.32 106.68) (end 157.48 106.68) (width 0.25) (layer B.Cu) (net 35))
 (segment (start 157.48 93.98) (end 154.94 93.98) (width 0.25) (layer B.Cu) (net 36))
 (segment (start 154.94 93.98) (end 154.94 104.14) (width 0.25) (layer B.Cu) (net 36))
 (segment (start 154.94 104.14) (end 147.32 104.14) (width 0.25) (layer B.Cu) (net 36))
 (segment (start 154.94 101.6) (end 154.94 86.36) (width 0.25) (layer F.Cu) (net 5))
 (segment (start 152.4 101.6) (end 154.94 101.6) (width 0.25) (layer F.Cu) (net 5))
 (segment (start 154.94 86.36) (end 157.48 86.36) (width 0.25) (layer B.Cu) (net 5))
 (via (at 154.94 86.36) (size 0.6) (drill 0.4) (layers F.Cu B.Cu) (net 5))
 (segment (start 149.86 101.6) (end 152.4 101.6) (width 0.25) (layer B.Cu) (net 5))
 (via (at 152.4 101.6) (size 0.6) (drill 0.4) (layers F.Cu B.Cu) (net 5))
 (segment (start 144.78 81.28) (end 144.78 73.66) (width 0.25) (layer B.Cu) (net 5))
 (segment (start 149.86 81.28) (end 144.78 81.28) (width 0.25) (layer B.Cu) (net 5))
 (segment (start 149.86 91.44) (end 149.86 81.28) (width 0.25) (layer B.Cu) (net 5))
 (segment (start 149.86 101.6) (end 149.86 91.44) (width 0.25) (layer F.Cu) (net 5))
 (via (at 149.86 91.44) (size 0.6) (drill 0.4) (layers F.Cu B.Cu) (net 5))
 (segment (start 147.32 101.6) (end 149.86 101.6) (width 0.25) (layer B.Cu) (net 5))
 (via (at 149.86 101.6) (size 0.6) (drill 0.4) (layers F.Cu B.Cu) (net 5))
 (segment (start 152.4 78.74) (end 157.48 78.74) (width 0.25) (layer B.Cu) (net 4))
 (segment (start 152.4 99.06) (end 152.4 78.74) (width 0.25) (layer B.Cu) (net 4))
 (segment (start 147.32 99.06) (end 152.4 99.06) (width 0.25) (layer B.Cu) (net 4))
 (segment (start 147.32 83.82) (end 147.32 99.06) (width 0.25) (layer B.Cu) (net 4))
 (segment (start 142.24 83.82) (end 147.32 83.82) (width 0.25) (layer B.Cu) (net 4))
 (segment (start 142.24 73.66) (end 142.24 83.82) (width 0.25) (layer B.Cu) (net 4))
 (segment (start 162.56 78.74) (end 160.02 78.74) (width 0.25) (layer B.Cu) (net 7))
 (segment (start 160.02 86.36) (end 162.56 86.36) (width 0.25) (layer B.Cu) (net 8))
 (segment (start 162.56 93.98) (end 160.02 93.98) (width 0.25) (layer B.Cu) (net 9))
 (segment (start 160.02 101.6) (end 162.56 101.6) (width 0.25) (layer B.Cu) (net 10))
 (segment (start 162.56 109.22) (end 160.02 109.22) (width 0.25) (layer B.Cu) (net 11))
 (segment (start 162.56 116.84) (end 160.02 116.84) (width 0.25) (layer B.Cu) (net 12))
 (segment (start 160.02 124.46) (end 162.56 124.46) (width 0.25) (layer B.Cu) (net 13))
 (segment (start 162.56 132.08) (end 160.02 132.08) (width 0.25) (layer B.Cu) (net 14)))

